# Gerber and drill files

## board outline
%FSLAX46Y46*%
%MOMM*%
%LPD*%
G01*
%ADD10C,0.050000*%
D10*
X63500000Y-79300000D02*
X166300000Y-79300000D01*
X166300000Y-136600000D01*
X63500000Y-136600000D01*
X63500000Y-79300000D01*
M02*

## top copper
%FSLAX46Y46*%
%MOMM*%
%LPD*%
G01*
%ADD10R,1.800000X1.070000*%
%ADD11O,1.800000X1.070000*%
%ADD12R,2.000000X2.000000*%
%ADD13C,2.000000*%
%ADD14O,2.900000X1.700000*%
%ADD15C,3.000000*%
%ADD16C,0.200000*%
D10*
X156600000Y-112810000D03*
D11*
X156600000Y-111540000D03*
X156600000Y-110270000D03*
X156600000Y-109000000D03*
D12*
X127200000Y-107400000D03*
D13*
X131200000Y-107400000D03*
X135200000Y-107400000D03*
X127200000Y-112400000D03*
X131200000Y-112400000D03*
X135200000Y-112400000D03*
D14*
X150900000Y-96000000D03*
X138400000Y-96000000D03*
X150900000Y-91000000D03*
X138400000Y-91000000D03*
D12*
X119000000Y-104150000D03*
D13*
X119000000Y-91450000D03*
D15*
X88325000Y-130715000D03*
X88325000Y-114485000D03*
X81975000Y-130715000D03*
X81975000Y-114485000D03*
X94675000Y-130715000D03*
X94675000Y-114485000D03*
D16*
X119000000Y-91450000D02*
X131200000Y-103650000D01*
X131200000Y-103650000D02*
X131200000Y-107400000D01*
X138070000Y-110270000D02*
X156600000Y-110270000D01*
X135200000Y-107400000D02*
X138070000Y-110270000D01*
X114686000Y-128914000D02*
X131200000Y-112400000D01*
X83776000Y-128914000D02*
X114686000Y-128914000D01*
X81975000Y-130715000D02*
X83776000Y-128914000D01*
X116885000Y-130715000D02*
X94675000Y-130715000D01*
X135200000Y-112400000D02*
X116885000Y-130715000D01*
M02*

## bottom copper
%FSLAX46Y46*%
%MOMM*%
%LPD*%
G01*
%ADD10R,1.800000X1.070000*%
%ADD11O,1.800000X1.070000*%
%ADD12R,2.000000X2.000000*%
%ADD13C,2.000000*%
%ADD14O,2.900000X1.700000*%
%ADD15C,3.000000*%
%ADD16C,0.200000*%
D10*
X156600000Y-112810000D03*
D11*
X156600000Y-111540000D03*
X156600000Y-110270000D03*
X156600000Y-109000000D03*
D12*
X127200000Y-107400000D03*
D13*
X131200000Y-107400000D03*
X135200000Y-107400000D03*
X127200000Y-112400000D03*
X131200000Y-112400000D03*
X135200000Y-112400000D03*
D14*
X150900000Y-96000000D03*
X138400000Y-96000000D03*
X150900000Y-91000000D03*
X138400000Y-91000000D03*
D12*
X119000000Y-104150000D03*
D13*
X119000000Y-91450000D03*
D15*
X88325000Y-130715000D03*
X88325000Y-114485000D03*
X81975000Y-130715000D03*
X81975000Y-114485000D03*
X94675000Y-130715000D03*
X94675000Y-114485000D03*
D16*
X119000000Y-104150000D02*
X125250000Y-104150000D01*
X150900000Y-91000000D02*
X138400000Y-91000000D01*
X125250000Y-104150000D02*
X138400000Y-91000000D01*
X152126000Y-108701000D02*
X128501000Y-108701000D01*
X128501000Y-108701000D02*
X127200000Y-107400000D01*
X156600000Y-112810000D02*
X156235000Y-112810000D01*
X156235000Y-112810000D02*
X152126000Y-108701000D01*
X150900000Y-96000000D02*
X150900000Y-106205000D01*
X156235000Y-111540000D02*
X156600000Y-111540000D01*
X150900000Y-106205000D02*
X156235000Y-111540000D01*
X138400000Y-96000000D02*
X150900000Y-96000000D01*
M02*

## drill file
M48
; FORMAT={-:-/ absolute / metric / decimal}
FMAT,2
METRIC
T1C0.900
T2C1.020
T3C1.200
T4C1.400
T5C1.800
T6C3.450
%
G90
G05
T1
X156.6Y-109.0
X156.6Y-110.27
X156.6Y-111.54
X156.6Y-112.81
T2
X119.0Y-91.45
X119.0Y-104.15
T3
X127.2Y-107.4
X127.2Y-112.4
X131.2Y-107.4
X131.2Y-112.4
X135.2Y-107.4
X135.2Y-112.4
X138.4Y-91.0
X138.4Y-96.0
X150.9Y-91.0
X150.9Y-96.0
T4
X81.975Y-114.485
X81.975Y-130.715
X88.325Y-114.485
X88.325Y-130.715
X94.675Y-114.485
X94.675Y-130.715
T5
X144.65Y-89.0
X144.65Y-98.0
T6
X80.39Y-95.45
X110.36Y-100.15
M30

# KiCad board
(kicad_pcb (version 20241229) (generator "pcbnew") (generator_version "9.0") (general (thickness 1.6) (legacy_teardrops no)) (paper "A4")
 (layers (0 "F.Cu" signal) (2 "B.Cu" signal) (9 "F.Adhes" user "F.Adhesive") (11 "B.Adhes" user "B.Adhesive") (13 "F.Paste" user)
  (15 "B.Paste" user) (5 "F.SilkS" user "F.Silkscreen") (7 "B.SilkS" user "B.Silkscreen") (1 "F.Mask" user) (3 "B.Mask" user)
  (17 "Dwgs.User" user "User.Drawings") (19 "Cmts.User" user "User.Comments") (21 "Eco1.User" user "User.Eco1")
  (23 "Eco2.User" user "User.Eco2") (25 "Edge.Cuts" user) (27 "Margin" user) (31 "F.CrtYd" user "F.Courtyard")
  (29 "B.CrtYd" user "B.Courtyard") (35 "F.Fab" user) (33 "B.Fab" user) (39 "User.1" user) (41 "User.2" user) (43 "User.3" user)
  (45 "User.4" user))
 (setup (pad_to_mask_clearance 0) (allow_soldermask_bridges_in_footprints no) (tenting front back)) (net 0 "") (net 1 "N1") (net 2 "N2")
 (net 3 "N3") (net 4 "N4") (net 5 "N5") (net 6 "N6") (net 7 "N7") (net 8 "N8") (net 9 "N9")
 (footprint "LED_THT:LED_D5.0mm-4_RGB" (layer "F.Cu") (at 156.6 112.81 90)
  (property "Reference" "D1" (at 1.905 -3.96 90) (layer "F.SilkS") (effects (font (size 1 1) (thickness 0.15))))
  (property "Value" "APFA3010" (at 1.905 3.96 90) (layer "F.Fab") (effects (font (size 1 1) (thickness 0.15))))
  (pad "1" thru_hole rect (at 0 0 90) (size 1.07 1.8) (drill 0.9) (layers "*.Cu" "*.Mask") (remove_unused_layers no) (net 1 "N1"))
  (pad "2" thru_hole oval (at 1.27 0 90) (size 1.07 1.8) (drill 0.9) (layers "*.Cu" "*.Mask") (remove_unused_layers no) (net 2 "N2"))
  (pad "3" thru_hole oval (at 2.54 0 90) (size 1.07 1.8) (drill 0.9) (layers "*.Cu" "*.Mask") (remove_unused_layers no) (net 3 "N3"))
  (pad "4" thru_hole oval (at 3.81 0 90) (size 1.07 1.8) (drill 0.9) (layers "*.Cu" "*.Mask") (remove_unused_layers no) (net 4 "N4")))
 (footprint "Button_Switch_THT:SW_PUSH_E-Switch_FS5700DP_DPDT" (layer "F.Cu") (at 127.2 107.4)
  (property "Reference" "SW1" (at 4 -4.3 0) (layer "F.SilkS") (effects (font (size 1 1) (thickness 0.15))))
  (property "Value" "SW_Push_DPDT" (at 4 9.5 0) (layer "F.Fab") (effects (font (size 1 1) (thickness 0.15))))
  (pad "1" thru_hole rect (at 0 0) (size 2 2) (drill 1.2) (layers "*.Cu" "*.Mask") (remove_unused_layers no) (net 1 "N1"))
  (pad "2" thru_hole circle (at 4 0) (size 2 2) (drill 1.2) (layers "*.Cu" "*.Mask") (remove_unused_layers no) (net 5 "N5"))
  (pad "3" thru_hole circle (at 8 0) (size 2 2) (drill 1.2) (layers "*.Cu" "*.Mask") (remove_unused_layers no) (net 3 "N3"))
  (pad "4" thru_hole circle (at 0 5) (size 2 2) (drill 1.2) (layers "*.Cu" "*.Mask") (remove_unused_layers no) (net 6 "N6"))
  (pad "5" thru_hole circle (at 4 5) (size 2 2) (drill 1.2) (layers "*.Cu" "*.Mask") (remove_unused_layers no) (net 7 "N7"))
  (pad "6" thru_hole circle (at 8 5) (size 2 2) (drill 1.2) (layers "*.Cu" "*.Mask") (remove_unused_layers no) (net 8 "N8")))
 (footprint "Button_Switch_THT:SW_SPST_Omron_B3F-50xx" (layer "F.Cu") (at 150.9 96 180)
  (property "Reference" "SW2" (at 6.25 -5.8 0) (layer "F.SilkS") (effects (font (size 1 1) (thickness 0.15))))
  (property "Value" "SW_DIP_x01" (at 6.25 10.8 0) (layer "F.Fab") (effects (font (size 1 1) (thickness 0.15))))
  (pad "" np_thru_hole circle (at 6.25 -2 180) (size 1.8 1.8) (drill 1.8) (layers "*.Cu" "*.Mask"))
  (pad "" np_thru_hole circle (at 6.25 7 180) (size 1.8 1.8) (drill 1.8) (layers "*.Cu" "*.Mask"))
  (pad "1" thru_hole oval (at 0 0 180) (size 2.9 1.7) (drill 1.2) (layers "*.Cu" "*.Mask") (remove_unused_layers no) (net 2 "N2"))
  (pad "1" thru_hole oval (at 12.5 0 180) (size 2.9 1.7) (drill 1.2) (layers "*.Cu" "*.Mask") (remove_unused_layers no) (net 2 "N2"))
  (pad "2" thru_hole oval (at 0 5 180) (size 2.9 1.7) (drill 1.2) (layers "*.Cu" "*.Mask") (remove_unused_layers no) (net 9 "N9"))
  (pad "2" thru_hole oval (at 12.5 5 180) (size 2.9 1.7) (drill 1.2) (layers "*.Cu" "*.Mask") (remove_unused_layers no) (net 9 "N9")))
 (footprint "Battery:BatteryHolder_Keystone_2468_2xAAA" (layer "F.Cu") (at 119 104.15 180)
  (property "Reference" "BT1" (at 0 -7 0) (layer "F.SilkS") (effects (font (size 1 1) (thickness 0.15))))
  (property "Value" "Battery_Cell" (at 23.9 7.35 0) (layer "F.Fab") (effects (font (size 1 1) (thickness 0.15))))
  (pad "" np_thru_hole circle (at 8.64 4 180) (size 3.45 3.45) (drill 3.45) (layers "*.Cu"))
  (pad "" np_thru_hole circle (at 38.61 8.7 180) (size 3.45 3.45) (drill 3.45) (layers "*.Cu" "*.Mask"))
  (pad "1" thru_hole rect (at 0 0 180) (size 2 2) (drill 1.02) (layers "*.Cu" "*.Mask") (remove_unused_layers no) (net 9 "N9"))
  (pad "2" thru_hole circle (at 0 12.7 180) (size 2 2) (drill 1.02) (layers "*.Cu" "*.Mask") (remove_unused_layers no) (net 5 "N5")))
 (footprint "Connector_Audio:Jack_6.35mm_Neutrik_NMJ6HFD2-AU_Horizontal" (layer "F.Cu") (at 94.675 130.715 180)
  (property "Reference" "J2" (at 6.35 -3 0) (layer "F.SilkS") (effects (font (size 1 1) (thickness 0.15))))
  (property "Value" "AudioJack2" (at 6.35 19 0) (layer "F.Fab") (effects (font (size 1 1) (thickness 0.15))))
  (pad "R" thru_hole circle (at 6.35 0 180) (size 3 3) (drill 1.4) (layers "*.Cu" "*.Mask") (remove_unused_layers no))
  (pad "RN" thru_hole circle (at 6.35 16.23 180) (size 3 3) (drill 1.4) (layers "*.Cu" "*.Mask") (remove_unused_layers no))
  (pad "S" thru_hole circle (at 12.7 0 180) (size 3 3) (drill 1.4) (layers "*.Cu" "*.Mask") (remove_unused_layers no) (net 7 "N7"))
  (pad "SN" thru_hole circle (at 12.7 16.23 180) (size 3 3) (drill 1.4) (layers "*.Cu" "*.Mask") (remove_unused_layers no))
  (pad "T" thru_hole circle (at 0 0 180) (size 3 3) (drill 1.4) (layers "*.Cu" "*.Mask") (remove_unused_layers no) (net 8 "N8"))
  (pad "TN" thru_hole circle (at 0 16.23 180) (size 3 3) (drill 1.4) (layers "*.Cu" "*.Mask") (remove_unused_layers no)))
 (gr_rect (start 63.5 79.3) (end 166.3 136.6) (stroke (width 0.05) (type default)) (fill no) (layer "Edge.Cuts"))
 (segment (start 119 91.45) (end 131.2 103.65) (width 0.2) (layer "F.Cu") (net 5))
 (segment (start 131.2 103.65) (end 131.2 107.4) (width 0.2) (layer "F.Cu") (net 5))
 (segment (start 119 104.15) (end 125.25 104.15) (width 0.2) (layer "B.Cu") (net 9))
 (segment (start 150.9 91) (end 138.4 91) (width 0.2) (layer "B.Cu") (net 9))
 (segment (start 125.25 104.15) (end 138.4 91) (width 0.2) (layer "B.Cu") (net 9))
 (segment (start 152.126 108.701) (end 128.501 108.701) (width 0.2) (layer "B.Cu") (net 1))
 (segment (start 128.501 108.701) (end 127.2 107.4) (width 0.2) (layer "B.Cu") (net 1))
 (segment (start 156.6 112.81) (end 156.235 112.81) (width 0.2) (layer "B.Cu") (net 1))
 (segment (start 156.235 112.81) (end 152.126 108.701) (width 0.2) (layer "B.Cu") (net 1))
 (segment (start 150.9 96) (end 150.9 106.205) (width 0.2) (layer "B.Cu") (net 2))
 (segment (start 156.235 111.54) (end 156.6 111.54) (width 0.2) (layer "B.Cu") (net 2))
 (segment (start 150.9 106.205) (end 156.235 111.54) (width 0.2) (layer "B.Cu") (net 2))
 (segment (start 138.4 96) (end 150.9 96) (width 0.2) (layer "B.Cu") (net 2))
 (segment (start 138.07 110.27) (end 156.6 110.27) (width 0.2) (layer "F.Cu") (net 3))
 (segment (start 135.2 107.4) (end 138.07 110.27) (width 0.2) (layer "F.Cu") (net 3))
 (segment (start 114.686 128.914) (end 131.2 112.4) (width 0.2) (layer "F.Cu") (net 7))
 (segment (start 83.776 128.914) (end 114.686 128.914) (width 0.2) (layer "F.Cu") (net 7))
 (segment (start 81.975 130.715) (end 83.776 128.914) (width 0.2) (layer "F.Cu") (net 7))
 (segment (start 116.885 130.715) (end 94.675 130.715) (width 0.2) (layer "F.Cu") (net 8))
 (segment (start 135.2 112.4) (end 116.885 130.715) (width 0.2) (layer "F.Cu") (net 8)))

